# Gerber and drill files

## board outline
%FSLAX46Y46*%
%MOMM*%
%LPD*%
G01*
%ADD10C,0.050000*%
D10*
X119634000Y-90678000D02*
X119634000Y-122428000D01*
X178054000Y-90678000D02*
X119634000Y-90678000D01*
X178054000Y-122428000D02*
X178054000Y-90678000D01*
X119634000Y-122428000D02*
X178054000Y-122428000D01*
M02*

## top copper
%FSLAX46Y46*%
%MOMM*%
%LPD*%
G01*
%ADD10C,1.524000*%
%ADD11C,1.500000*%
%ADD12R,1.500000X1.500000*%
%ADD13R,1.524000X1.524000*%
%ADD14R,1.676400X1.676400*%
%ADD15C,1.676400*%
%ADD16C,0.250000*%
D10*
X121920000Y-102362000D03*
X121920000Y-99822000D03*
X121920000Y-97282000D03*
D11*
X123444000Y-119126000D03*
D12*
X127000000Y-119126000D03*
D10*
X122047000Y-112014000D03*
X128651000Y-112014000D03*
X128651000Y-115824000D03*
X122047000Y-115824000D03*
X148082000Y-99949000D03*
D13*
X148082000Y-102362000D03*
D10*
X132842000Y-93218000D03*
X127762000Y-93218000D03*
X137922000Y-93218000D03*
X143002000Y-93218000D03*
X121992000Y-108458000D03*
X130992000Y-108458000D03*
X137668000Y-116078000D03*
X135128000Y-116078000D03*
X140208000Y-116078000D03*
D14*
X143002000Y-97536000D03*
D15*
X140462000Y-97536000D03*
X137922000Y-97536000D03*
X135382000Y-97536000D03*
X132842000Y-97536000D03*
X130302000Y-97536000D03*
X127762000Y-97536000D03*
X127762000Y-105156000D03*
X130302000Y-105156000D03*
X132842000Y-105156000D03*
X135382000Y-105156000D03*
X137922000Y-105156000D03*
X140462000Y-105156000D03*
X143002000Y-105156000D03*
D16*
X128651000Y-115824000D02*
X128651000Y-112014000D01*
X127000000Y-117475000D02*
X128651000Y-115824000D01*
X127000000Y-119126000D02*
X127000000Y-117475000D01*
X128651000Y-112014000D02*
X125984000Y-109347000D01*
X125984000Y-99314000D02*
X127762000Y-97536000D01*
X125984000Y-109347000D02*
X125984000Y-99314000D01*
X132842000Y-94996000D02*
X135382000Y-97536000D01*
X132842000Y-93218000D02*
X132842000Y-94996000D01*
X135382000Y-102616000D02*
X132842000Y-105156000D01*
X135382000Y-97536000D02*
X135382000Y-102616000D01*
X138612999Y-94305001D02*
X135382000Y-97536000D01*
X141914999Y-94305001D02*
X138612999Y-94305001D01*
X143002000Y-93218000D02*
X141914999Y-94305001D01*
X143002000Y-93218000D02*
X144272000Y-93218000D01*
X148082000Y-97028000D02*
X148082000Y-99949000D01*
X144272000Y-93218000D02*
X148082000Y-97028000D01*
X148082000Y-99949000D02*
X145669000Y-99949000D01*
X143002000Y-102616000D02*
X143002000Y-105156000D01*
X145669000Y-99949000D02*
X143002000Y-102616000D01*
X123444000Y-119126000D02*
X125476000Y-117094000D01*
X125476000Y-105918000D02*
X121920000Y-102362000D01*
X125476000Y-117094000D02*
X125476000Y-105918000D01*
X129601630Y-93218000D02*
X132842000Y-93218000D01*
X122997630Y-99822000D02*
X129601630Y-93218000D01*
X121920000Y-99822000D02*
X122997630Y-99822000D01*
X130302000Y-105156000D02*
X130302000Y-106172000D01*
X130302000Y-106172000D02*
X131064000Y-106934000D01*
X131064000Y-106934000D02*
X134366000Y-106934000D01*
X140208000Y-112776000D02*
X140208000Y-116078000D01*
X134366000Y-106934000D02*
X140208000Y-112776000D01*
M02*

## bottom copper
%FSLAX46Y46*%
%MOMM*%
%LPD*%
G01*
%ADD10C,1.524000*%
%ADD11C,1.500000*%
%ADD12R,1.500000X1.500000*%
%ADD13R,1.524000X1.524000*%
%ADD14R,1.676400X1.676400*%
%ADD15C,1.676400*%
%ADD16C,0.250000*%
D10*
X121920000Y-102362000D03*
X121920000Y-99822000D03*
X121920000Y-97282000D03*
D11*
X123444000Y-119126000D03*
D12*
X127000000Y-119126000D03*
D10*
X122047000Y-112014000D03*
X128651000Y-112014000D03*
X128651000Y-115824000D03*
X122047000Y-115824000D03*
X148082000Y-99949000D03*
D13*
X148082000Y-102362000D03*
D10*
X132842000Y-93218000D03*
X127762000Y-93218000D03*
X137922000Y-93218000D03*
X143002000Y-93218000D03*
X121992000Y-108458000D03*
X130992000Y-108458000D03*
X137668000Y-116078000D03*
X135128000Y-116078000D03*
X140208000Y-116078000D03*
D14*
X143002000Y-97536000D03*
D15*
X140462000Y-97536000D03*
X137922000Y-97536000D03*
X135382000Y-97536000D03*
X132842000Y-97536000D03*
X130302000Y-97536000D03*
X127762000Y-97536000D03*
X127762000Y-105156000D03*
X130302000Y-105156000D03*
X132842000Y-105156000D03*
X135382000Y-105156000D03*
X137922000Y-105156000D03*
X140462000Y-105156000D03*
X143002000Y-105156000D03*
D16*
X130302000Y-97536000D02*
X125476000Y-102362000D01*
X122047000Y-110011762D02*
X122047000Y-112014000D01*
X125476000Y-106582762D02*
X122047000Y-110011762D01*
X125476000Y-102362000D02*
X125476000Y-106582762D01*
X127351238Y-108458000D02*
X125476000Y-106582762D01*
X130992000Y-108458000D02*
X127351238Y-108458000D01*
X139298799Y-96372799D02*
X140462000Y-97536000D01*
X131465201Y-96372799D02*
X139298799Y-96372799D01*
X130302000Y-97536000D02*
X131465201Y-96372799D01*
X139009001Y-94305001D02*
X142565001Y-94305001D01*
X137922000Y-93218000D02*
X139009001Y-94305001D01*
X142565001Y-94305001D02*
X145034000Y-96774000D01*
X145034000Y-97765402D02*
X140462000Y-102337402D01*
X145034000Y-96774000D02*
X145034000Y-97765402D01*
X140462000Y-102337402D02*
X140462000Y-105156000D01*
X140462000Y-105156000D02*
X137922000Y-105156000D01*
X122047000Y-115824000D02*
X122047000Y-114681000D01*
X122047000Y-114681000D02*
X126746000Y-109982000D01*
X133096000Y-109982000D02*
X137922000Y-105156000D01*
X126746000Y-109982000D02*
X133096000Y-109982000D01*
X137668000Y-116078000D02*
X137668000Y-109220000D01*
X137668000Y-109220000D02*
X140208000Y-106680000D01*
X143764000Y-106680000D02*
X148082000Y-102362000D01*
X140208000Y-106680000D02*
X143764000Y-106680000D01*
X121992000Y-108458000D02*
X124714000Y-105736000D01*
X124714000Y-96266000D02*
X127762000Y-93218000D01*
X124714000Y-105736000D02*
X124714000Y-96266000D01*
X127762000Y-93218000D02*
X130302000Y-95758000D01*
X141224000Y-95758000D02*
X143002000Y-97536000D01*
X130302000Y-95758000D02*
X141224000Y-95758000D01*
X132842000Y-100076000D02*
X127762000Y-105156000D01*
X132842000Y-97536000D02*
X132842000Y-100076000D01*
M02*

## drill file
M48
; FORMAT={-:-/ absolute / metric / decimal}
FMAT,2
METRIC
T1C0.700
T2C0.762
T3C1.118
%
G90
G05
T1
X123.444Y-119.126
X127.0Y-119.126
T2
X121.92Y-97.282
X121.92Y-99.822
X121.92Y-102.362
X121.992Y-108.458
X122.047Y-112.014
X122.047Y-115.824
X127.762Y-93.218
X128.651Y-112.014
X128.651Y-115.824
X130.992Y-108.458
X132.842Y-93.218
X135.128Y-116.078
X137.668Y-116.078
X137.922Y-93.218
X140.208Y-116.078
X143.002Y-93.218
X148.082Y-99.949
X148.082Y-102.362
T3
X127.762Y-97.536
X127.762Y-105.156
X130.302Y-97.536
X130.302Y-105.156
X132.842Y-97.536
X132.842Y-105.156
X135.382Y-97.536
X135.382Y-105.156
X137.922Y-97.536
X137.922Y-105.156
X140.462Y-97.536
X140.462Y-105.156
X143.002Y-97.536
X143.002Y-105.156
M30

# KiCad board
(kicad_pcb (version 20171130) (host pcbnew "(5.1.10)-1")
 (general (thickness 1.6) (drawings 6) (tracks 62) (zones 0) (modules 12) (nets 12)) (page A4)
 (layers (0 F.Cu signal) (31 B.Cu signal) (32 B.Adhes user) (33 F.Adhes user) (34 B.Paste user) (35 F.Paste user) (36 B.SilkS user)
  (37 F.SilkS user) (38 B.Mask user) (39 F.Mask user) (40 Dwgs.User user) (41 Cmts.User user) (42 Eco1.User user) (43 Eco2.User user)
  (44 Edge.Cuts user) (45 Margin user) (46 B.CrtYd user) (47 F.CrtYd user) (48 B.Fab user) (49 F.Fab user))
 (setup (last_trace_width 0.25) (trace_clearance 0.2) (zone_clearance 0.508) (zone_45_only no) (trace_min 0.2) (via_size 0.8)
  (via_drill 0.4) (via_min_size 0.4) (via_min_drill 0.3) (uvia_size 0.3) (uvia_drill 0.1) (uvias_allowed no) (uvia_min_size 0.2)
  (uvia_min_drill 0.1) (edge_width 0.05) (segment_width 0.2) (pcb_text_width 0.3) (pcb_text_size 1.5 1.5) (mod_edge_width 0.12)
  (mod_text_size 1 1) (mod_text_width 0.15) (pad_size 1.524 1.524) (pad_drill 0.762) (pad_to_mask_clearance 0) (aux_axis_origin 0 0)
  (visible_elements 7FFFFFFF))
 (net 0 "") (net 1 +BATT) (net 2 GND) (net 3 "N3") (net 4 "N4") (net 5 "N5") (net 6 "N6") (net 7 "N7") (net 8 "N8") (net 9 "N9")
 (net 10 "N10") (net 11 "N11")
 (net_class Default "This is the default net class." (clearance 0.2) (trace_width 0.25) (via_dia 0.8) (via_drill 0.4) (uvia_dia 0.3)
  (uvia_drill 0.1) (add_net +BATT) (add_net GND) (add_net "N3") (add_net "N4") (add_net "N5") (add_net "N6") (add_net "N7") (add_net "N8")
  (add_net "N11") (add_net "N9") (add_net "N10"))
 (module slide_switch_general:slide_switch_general (layer F.Cu) (at 121.92 99.822 270)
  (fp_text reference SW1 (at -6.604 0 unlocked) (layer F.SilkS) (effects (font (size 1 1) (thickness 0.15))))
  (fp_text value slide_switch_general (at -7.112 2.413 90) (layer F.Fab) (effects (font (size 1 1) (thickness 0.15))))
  (pad 3 thru_hole circle (at 2.54 0 270) (size 1.524 1.524) (drill 0.762) (layers *.Cu *.Mask) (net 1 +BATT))
  (pad 2 thru_hole circle (at 0 0 270) (size 1.524 1.524) (drill 0.762) (layers *.Cu *.Mask) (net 1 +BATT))
  (pad 1 thru_hole circle (at -2.54 0 270) (size 1.524 1.524) (drill 0.762) (layers *.Cu *.Mask)))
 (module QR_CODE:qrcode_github (layer F.Cu) (at 166.37 102.108)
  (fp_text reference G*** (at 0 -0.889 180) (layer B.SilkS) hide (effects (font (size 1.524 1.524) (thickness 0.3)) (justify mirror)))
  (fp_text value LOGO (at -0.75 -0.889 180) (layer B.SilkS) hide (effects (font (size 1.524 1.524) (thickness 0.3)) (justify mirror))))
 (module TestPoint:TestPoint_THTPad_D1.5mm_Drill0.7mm (layer F.Cu) (at 123.444 119.126)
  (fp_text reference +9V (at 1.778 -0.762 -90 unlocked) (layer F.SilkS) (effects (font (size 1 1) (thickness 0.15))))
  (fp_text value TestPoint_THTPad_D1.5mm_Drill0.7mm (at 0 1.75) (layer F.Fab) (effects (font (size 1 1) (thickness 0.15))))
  (pad 1 thru_hole circle (at 0 0) (size 1.5 1.5) (drill 0.7) (layers *.Cu *.Mask) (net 1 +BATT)))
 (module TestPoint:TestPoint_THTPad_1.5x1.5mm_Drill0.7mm (layer F.Cu) (at 127 119.126)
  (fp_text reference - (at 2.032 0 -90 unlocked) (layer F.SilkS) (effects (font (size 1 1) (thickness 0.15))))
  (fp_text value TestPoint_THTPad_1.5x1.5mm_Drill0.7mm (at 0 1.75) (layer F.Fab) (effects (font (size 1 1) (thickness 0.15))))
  (pad 1 thru_hole rect (at 0 0) (size 1.5 1.5) (drill 0.7) (layers *.Cu *.Mask) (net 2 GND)))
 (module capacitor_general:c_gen (layer F.Cu) (at 125.476 112.014)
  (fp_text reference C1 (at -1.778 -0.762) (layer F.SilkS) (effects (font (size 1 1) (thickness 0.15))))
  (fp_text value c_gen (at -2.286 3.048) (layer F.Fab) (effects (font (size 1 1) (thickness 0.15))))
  (pad 1 thru_hole circle (at -3.429 0) (size 1.524 1.524) (drill 0.762) (layers *.Cu *.Mask) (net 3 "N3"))
  (pad 2 thru_hole circle (at 3.175 0) (size 1.524 1.524) (drill 0.762) (layers *.Cu *.Mask) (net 2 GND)))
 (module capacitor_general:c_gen (layer F.Cu) (at 125.476 115.824)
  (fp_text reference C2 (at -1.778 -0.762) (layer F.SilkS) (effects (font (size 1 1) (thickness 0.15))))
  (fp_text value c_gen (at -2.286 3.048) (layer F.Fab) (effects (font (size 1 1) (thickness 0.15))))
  (pad 2 thru_hole circle (at 3.175 0) (size 1.524 1.524) (drill 0.762) (layers *.Cu *.Mask) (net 2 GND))
  (pad 1 thru_hole circle (at -3.429 0) (size 1.524 1.524) (drill 0.762) (layers *.Cu *.Mask) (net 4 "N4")))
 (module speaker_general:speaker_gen (layer F.Cu) (at 148.082 101.092 270)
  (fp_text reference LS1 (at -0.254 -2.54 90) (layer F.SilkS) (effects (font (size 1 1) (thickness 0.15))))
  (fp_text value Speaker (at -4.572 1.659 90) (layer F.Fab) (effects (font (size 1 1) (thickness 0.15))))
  (pad 1 thru_hole circle (at -1.143 0 270) (size 1.524 1.524) (drill 0.762) (layers *.Cu *.Mask) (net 1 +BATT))
  (pad 2 thru_hole rect (at 1.27 0 270) (size 1.524 1.524) (drill 0.762) (layers *.Cu *.Mask) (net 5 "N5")))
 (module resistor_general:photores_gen (layer F.Cu) (at 130.302 93.218 180)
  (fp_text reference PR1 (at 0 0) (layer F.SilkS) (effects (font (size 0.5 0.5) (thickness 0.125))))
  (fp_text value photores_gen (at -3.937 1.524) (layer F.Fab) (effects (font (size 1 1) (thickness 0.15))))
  (pad 1 thru_hole circle (at -2.54 0 180) (size 1.524 1.524) (drill 0.762) (layers *.Cu *.Mask) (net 1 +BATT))
  (pad 2 thru_hole circle (at 2.54 0 180) (size 1.524 1.524) (drill 0.762) (layers *.Cu *.Mask) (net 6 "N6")))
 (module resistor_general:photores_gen (layer F.Cu) (at 140.462 93.218 180)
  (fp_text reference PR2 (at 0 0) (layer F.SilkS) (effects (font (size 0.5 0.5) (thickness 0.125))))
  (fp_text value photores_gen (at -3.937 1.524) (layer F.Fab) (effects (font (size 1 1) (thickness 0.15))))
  (pad 2 thru_hole circle (at 2.54 0 180) (size 1.524 1.524) (drill 0.762) (layers *.Cu *.Mask) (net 4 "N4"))
  (pad 1 thru_hole circle (at -2.54 0 180) (size 1.524 1.524) (drill 0.762) (layers *.Cu *.Mask) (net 1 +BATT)))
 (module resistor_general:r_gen (layer F.Cu) (at 126.492 108.458)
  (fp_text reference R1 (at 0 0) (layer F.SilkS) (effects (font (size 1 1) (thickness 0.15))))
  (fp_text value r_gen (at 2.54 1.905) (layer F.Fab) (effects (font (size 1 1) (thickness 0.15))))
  (pad 1 thru_hole circle (at -4.5 0) (size 1.524 1.524) (drill 0.762) (layers *.Cu *.Mask) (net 6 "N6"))
  (pad 2 thru_hole circle (at 4.5 0) (size 1.524 1.524) (drill 0.762) (layers *.Cu *.Mask) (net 3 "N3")))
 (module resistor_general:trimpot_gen (layer F.Cu) (at 137.668 117.094)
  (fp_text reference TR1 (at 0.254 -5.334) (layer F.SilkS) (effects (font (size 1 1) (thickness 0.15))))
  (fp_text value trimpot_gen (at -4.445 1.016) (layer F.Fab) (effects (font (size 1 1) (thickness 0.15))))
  (pad 2 thru_hole circle (at 0 -1.016) (size 1.524 1.524) (drill 0.762) (layers *.Cu *.Mask) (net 5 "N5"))
  (pad 1 thru_hole circle (at -2.54 -1.016) (size 1.524 1.524) (drill 0.762) (layers *.Cu *.Mask) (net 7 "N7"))
  (pad 3 thru_hole circle (at 2.54 -1.016) (size 1.524 1.524) (drill 0.762) (layers *.Cu *.Mask) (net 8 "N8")))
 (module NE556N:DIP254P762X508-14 (layer F.Cu) (at 127.762 105.156 270)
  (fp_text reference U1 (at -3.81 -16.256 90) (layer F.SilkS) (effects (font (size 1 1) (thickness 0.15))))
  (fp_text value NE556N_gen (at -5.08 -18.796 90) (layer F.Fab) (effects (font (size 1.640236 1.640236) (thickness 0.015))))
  (pad 1 thru_hole rect (at -7.62 -15.24 270) (size 1.6764 1.6764) (drill 1.1176) (layers *.Cu *.Mask) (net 6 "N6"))
  (pad 2 thru_hole circle (at -7.62 -12.7 270) (size 1.6764 1.6764) (drill 1.1176) (layers *.Cu *.Mask) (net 3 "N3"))
  (pad 3 thru_hole circle (at -7.62 -10.16 270) (size 1.6764 1.6764) (drill 1.1176) (layers *.Cu *.Mask) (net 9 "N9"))
  (pad 4 thru_hole circle (at -7.62 -7.62 270) (size 1.6764 1.6764) (drill 1.1176) (layers *.Cu *.Mask) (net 1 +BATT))
  (pad 5 thru_hole circle (at -7.62 -5.08 270) (size 1.6764 1.6764) (drill 1.1176) (layers *.Cu *.Mask) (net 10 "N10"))
  (pad 6 thru_hole circle (at -7.62 -2.54 270) (size 1.6764 1.6764) (drill 1.1176) (layers *.Cu *.Mask) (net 3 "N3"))
  (pad 7 thru_hole circle (at -7.62 0 270) (size 1.6764 1.6764) (drill 1.1176) (layers *.Cu *.Mask) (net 2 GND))
  (pad 8 thru_hole circle (at 0 0 270) (size 1.6764 1.6764) (drill 1.1176) (layers *.Cu *.Mask) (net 10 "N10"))
  (pad 9 thru_hole circle (at 0 -2.54 270) (size 1.6764 1.6764) (drill 1.1176) (layers *.Cu *.Mask) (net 8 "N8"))
  (pad 10 thru_hole circle (at 0 -5.08 270) (size 1.6764 1.6764) (drill 1.1176) (layers *.Cu *.Mask) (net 1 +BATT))
  (pad 11 thru_hole circle (at 0 -7.62 270) (size 1.6764 1.6764) (drill 1.1176) (layers *.Cu *.Mask) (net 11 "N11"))
  (pad 12 thru_hole circle (at 0 -10.16 270) (size 1.6764 1.6764) (drill 1.1176) (layers *.Cu *.Mask) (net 4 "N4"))
  (pad 13 thru_hole circle (at 0 -12.7 270) (size 1.6764 1.6764) (drill 1.1176) (layers *.Cu *.Mask) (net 4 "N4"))
  (pad 14 thru_hole circle (at 0 -15.24 270) (size 1.6764 1.6764) (drill 1.1176) (layers *.Cu *.Mask) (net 1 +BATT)))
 (gr_line (start 119.634 90.678) (end 119.634 122.428) (layer Edge.Cuts) (width 0.05))
 (gr_line (start 178.054 90.678) (end 119.634 90.678) (layer Edge.Cuts) (width 0.05))
 (gr_line (start 178.054 122.428) (end 178.054 90.678) (layer Edge.Cuts) (width 0.05))
 (gr_line (start 119.634 122.428) (end 178.054 122.428) (layer Edge.Cuts) (width 0.05))
 (segment (start 130.302 97.536) (end 125.476 102.362) (width 0.25) (layer B.Cu) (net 3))
 (segment (start 122.047 110.011762) (end 122.047 112.014) (width 0.25) (layer B.Cu) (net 3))
 (segment (start 125.476 106.582762) (end 122.047 110.011762) (width 0.25) (layer B.Cu) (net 3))
 (segment (start 125.476 102.362) (end 125.476 106.582762) (width 0.25) (layer B.Cu) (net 3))
 (segment (start 127.351238 108.458) (end 125.476 106.582762) (width 0.25) (layer B.Cu) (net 3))
 (segment (start 130.992 108.458) (end 127.351238 108.458) (width 0.25) (layer B.Cu) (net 3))
 (segment (start 139.298799 96.372799) (end 140.462 97.536) (width 0.25) (layer B.Cu) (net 3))
 (segment (start 131.465201 96.372799) (end 139.298799 96.372799) (width 0.25) (layer B.Cu) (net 3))
 (segment (start 130.302 97.536) (end 131.465201 96.372799) (width 0.25) (layer B.Cu) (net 3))
 (segment (start 128.651 115.824) (end 128.651 112.014) (width 0.25) (layer F.Cu) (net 2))
 (segment (start 127 117.475) (end 128.651 115.824) (width 0.25) (layer F.Cu) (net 2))
 (segment (start 127 119.126) (end 127 117.475) (width 0.25) (layer F.Cu) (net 2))
 (segment (start 128.651 112.014) (end 125.984 109.347) (width 0.25) (layer F.Cu) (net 2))
 (segment (start 125.984 99.314) (end 127.762 97.536) (width 0.25) (layer F.Cu) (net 2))
 (segment (start 125.984 109.347) (end 125.984 99.314) (width 0.25) (layer F.Cu) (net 2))
 (segment (start 139.009001 94.305001) (end 142.565001 94.305001) (width 0.25) (layer B.Cu) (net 4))
 (segment (start 137.922 93.218) (end 139.009001 94.305001) (width 0.25) (layer B.Cu) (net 4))
 (segment (start 142.565001 94.305001) (end 145.034 96.774) (width 0.25) (layer B.Cu) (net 4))
 (segment (start 145.034 97.765402) (end 140.462 102.337402) (width 0.25) (layer B.Cu) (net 4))
 (segment (start 145.034 96.774) (end 145.034 97.765402) (width 0.25) (layer B.Cu) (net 4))
 (segment (start 140.462 102.337402) (end 140.462 105.156) (width 0.25) (layer B.Cu) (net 4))
 (segment (start 140.462 105.156) (end 137.922 105.156) (width 0.25) (layer B.Cu) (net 4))
 (segment (start 122.047 115.824) (end 122.047 114.681) (width 0.25) (layer B.Cu) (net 4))
 (segment (start 122.047 114.681) (end 126.746 109.982) (width 0.25) (layer B.Cu) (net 4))
 (segment (start 133.096 109.982) (end 137.922 105.156) (width 0.25) (layer B.Cu) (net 4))
 (segment (start 126.746 109.982) (end 133.096 109.982) (width 0.25) (layer B.Cu) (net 4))
 (segment (start 132.842 94.996) (end 135.382 97.536) (width 0.25) (layer F.Cu) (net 1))
 (segment (start 132.842 93.218) (end 132.842 94.996) (width 0.25) (layer F.Cu) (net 1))
 (segment (start 135.382 102.616) (end 132.842 105.156) (width 0.25) (layer F.Cu) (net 1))
 (segment (start 135.382 97.536) (end 135.382 102.616) (width 0.25) (layer F.Cu) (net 1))
 (segment (start 138.612999 94.305001) (end 135.382 97.536) (width 0.25) (layer F.Cu) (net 1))
 (segment (start 141.914999 94.305001) (end 138.612999 94.305001) (width 0.25) (layer F.Cu) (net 1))
 (segment (start 143.002 93.218) (end 141.914999 94.305001) (width 0.25) (layer F.Cu) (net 1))
 (segment (start 143.002 93.218) (end 144.272 93.218) (width 0.25) (layer F.Cu) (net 1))
 (segment (start 148.082 97.028) (end 148.082 99.949) (width 0.25) (layer F.Cu) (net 1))
 (segment (start 144.272 93.218) (end 148.082 97.028) (width 0.25) (layer F.Cu) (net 1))
 (segment (start 148.082 99.949) (end 145.669 99.949) (width 0.25) (layer F.Cu) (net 1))
 (segment (start 143.002 102.616) (end 143.002 105.156) (width 0.25) (layer F.Cu) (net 1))
 (segment (start 145.669 99.949) (end 143.002 102.616) (width 0.25) (layer F.Cu) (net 1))
 (segment (start 123.444 119.126) (end 125.476 117.094) (width 0.25) (layer F.Cu) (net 1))
 (segment (start 125.476 105.918) (end 121.92 102.362) (width 0.25) (layer F.Cu) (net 1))
 (segment (start 125.476 117.094) (end 125.476 105.918) (width 0.25) (layer F.Cu) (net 1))
 (segment (start 129.60163 93.218) (end 132.842 93.218) (width 0.25) (layer F.Cu) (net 1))
 (segment (start 122.99763 99.822) (end 129.60163 93.218) (width 0.25) (layer F.Cu) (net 1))
 (segment (start 121.92 99.822) (end 122.99763 99.822) (width 0.25) (layer F.Cu) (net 1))
 (segment (start 137.668 116.078) (end 137.668 109.22) (width 0.25) (layer B.Cu) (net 5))
 (segment (start 137.668 109.22) (end 140.208 106.68) (width 0.25) (layer B.Cu) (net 5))
 (segment (start 143.764 106.68) (end 148.082 102.362) (width 0.25) (layer B.Cu) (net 5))
 (segment (start 140.208 106.68) (end 143.764 106.68) (width 0.25) (layer B.Cu) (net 5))
 (segment (start 121.992 108.458) (end 124.714 105.736) (width 0.25) (layer B.Cu) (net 6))
 (segment (start 124.714 96.266) (end 127.762 93.218) (width 0.25) (layer B.Cu) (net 6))
 (segment (start 124.714 105.736) (end 124.714 96.266) (width 0.25) (layer B.Cu) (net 6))
 (segment (start 127.762 93.218) (end 130.302 95.758) (width 0.25) (layer B.Cu) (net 6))
 (segment (start 141.224 95.758) (end 143.002 97.536) (width 0.25) (layer B.Cu) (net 6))
 (segment (start 130.302 95.758) (end 141.224 95.758) (width 0.25) (layer B.Cu) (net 6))
 (segment (start 130.302 105.156) (end 130.302 106.172) (width 0.25) (layer F.Cu) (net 8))
 (segment (start 130.302 106.172) (end 131.064 106.934) (width 0.25) (layer F.Cu) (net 8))
 (segment (start 131.064 106.934) (end 134.366 106.934) (width 0.25) (layer F.Cu) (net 8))
 (segment (start 140.208 112.776) (end 140.208 116.078) (width 0.25) (layer F.Cu) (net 8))
 (segment (start 134.366 106.934) (end 140.208 112.776) (width 0.25) (layer F.Cu) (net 8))
 (segment (start 132.842 100.076) (end 127.762 105.156) (width 0.25) (layer B.Cu) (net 10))
 (segment (start 132.842 97.536) (end 132.842 100.076) (width 0.25) (layer B.Cu) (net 10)))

